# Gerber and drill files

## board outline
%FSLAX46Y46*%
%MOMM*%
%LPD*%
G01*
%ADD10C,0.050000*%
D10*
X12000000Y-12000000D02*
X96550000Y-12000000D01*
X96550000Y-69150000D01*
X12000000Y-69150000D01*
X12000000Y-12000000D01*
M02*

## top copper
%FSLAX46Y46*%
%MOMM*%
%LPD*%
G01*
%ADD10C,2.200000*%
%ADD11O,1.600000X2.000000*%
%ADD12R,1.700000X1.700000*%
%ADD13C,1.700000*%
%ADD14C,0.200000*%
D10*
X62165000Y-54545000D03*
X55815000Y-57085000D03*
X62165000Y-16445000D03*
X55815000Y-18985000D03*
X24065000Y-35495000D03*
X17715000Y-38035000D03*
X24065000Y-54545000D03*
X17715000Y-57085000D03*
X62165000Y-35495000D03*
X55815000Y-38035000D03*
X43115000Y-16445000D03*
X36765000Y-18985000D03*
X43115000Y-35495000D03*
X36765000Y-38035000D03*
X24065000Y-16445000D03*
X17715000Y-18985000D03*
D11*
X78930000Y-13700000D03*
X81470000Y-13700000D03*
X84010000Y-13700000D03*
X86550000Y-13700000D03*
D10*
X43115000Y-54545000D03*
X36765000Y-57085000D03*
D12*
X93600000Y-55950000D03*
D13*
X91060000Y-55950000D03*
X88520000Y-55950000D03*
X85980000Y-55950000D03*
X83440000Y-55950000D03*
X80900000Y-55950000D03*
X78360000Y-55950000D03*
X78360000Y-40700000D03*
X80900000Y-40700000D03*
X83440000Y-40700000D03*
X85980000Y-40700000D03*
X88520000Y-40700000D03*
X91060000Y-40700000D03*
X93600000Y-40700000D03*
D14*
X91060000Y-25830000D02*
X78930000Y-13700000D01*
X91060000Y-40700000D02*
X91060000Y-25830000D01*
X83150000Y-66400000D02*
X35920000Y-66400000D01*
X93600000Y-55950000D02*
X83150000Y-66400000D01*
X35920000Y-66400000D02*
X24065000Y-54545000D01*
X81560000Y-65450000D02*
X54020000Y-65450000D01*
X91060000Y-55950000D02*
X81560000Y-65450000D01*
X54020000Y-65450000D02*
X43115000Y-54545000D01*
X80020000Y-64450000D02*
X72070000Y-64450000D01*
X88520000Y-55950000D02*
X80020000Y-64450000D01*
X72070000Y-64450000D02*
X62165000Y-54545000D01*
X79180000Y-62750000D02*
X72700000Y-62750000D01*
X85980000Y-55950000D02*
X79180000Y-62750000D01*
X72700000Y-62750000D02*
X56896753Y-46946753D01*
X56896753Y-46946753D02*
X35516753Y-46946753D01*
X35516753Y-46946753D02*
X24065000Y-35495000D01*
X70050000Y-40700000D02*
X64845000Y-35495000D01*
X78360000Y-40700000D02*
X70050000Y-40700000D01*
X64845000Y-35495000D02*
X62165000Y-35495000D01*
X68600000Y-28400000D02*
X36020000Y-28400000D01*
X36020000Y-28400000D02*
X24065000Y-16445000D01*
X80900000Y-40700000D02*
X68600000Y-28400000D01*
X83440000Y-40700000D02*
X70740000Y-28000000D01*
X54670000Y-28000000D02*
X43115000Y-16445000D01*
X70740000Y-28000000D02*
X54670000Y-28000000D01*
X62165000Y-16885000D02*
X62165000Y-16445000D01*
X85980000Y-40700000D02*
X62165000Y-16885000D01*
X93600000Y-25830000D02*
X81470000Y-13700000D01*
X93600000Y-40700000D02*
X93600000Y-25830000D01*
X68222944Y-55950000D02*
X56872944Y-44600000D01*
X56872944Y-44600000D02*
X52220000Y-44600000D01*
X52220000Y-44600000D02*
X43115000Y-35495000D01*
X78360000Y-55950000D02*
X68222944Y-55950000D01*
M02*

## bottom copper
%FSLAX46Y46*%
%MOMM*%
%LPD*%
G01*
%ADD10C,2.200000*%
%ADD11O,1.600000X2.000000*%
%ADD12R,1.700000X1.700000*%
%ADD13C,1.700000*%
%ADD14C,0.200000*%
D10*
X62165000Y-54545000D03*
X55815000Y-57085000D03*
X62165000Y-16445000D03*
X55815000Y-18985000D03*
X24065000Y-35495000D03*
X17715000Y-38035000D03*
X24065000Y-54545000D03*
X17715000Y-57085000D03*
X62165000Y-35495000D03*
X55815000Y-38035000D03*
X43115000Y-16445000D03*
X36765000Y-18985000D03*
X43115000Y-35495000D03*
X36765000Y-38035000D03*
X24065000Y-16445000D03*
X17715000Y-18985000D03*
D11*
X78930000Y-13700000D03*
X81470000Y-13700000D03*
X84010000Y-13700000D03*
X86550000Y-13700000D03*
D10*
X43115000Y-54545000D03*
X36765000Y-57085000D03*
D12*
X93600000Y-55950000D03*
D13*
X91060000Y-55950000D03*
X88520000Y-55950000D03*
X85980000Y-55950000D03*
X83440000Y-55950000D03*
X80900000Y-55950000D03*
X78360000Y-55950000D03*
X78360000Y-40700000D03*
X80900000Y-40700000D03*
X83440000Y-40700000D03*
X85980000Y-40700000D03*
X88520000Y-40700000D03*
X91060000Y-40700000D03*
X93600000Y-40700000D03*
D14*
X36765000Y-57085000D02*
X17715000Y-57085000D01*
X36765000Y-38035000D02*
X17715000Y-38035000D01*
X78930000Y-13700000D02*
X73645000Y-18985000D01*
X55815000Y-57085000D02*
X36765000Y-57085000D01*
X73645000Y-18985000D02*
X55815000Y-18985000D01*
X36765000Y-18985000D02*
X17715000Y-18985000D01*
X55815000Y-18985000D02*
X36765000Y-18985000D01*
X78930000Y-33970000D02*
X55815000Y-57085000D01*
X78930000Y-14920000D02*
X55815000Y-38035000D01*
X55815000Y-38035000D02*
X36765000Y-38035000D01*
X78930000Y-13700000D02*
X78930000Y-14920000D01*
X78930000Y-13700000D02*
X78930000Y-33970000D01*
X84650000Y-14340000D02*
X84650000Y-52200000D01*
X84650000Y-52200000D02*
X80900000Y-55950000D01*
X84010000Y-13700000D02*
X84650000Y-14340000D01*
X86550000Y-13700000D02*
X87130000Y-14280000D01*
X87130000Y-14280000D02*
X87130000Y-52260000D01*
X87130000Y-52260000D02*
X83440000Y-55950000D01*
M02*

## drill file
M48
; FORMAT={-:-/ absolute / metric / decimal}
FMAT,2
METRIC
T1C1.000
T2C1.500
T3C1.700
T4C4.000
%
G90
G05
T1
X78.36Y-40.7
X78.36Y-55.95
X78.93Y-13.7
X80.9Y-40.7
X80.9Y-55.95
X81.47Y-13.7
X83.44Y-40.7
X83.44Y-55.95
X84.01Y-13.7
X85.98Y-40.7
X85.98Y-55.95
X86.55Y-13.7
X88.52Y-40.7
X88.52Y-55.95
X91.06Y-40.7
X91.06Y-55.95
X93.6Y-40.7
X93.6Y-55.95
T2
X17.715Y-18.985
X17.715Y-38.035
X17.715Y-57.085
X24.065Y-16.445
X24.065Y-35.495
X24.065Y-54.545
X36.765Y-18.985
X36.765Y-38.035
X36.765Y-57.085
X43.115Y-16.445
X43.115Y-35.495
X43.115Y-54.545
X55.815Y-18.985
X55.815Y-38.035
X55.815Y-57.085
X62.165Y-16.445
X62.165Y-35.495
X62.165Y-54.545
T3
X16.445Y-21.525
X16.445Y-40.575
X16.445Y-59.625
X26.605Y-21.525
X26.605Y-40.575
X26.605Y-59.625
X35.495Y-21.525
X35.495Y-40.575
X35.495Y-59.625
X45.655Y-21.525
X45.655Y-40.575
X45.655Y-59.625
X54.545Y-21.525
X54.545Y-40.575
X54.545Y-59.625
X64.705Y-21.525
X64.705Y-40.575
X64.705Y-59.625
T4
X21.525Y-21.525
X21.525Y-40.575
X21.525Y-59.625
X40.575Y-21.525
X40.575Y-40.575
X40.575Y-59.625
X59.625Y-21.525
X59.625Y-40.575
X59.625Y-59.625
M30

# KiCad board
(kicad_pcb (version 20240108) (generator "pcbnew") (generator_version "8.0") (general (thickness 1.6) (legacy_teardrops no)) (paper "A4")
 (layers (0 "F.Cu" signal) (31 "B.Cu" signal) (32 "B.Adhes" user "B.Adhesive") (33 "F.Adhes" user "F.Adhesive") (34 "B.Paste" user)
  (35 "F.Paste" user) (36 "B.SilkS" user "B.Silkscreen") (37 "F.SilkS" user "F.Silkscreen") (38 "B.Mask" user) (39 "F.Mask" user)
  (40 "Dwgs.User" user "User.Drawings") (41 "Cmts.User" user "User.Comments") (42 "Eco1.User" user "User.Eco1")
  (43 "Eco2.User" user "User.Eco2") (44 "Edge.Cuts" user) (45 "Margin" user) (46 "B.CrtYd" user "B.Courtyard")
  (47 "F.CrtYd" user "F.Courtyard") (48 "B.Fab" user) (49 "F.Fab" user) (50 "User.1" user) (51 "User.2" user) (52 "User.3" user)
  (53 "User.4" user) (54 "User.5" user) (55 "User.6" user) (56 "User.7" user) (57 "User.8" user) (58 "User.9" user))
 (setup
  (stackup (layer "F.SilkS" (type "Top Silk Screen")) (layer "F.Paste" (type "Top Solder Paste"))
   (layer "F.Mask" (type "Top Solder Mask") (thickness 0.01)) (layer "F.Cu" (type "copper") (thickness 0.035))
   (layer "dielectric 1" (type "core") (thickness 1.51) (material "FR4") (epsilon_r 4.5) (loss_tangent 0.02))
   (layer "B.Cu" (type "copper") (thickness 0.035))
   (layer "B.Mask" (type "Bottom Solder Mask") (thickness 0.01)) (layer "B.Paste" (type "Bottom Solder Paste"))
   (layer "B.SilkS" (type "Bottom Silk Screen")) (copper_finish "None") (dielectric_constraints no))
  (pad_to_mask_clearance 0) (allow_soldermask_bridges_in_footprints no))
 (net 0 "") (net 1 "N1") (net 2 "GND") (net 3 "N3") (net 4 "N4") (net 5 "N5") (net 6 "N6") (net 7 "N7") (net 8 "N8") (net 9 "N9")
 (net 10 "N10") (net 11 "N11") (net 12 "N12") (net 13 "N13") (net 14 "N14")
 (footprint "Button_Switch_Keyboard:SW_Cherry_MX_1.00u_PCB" (layer "F.Cu") (at 62.165 54.545)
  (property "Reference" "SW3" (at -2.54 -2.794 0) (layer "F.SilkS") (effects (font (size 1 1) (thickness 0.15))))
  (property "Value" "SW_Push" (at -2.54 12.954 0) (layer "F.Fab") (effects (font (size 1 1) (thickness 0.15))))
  (pad "" np_thru_hole circle (at -7.62 5.08) (size 1.7 1.7) (drill 1.7) (layers "*.Cu" "*.Mask"))
  (pad "" np_thru_hole circle (at -2.54 5.08) (size 4 4) (drill 4) (layers "*.Cu" "*.Mask"))
  (pad "" np_thru_hole circle (at 2.54 5.08) (size 1.7 1.7) (drill 1.7) (layers "*.Cu" "*.Mask"))
  (pad "1" thru_hole circle (at 0 0) (size 2.2 2.2) (drill 1.5) (layers "*.Cu" "*.Mask") (remove_unused_layers no) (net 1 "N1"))
  (pad "2" thru_hole circle (at -6.35 2.54) (size 2.2 2.2) (drill 1.5) (layers "*.Cu" "*.Mask") (remove_unused_layers no) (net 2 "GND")))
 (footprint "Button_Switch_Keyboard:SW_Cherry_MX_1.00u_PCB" (layer "F.Cu") (at 62.165 16.445)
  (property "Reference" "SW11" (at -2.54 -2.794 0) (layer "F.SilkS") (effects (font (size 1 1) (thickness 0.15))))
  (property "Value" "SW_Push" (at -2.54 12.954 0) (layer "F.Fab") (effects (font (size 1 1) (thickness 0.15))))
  (pad "" np_thru_hole circle (at -7.62 5.08) (size 1.7 1.7) (drill 1.7) (layers "*.Cu" "*.Mask"))
  (pad "" np_thru_hole circle (at -2.54 5.08) (size 4 4) (drill 4) (layers "*.Cu" "*.Mask"))
  (pad "" np_thru_hole circle (at 2.54 5.08) (size 1.7 1.7) (drill 1.7) (layers "*.Cu" "*.Mask"))
  (pad "1" thru_hole circle (at 0 0) (size 2.2 2.2) (drill 1.5) (layers "*.Cu" "*.Mask") (remove_unused_layers no) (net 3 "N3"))
  (pad "2" thru_hole circle (at -6.35 2.54) (size 2.2 2.2) (drill 1.5) (layers "*.Cu" "*.Mask") (remove_unused_layers no) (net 2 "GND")))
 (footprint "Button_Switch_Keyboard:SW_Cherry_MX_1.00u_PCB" (layer "F.Cu") (at 24.065 35.495)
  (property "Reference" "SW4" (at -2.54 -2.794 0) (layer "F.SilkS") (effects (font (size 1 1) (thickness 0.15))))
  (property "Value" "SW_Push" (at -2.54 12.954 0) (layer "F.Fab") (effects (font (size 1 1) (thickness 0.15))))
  (pad "" np_thru_hole circle (at -7.62 5.08) (size 1.7 1.7) (drill 1.7) (layers "*.Cu" "*.Mask"))
  (pad "" np_thru_hole circle (at -2.54 5.08) (size 4 4) (drill 4) (layers "*.Cu" "*.Mask"))
  (pad "" np_thru_hole circle (at 2.54 5.08) (size 1.7 1.7) (drill 1.7) (layers "*.Cu" "*.Mask"))
  (pad "1" thru_hole circle (at 0 0) (size 2.2 2.2) (drill 1.5) (layers "*.Cu" "*.Mask") (remove_unused_layers no) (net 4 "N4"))
  (pad "2" thru_hole circle (at -6.35 2.54) (size 2.2 2.2) (drill 1.5) (layers "*.Cu" "*.Mask") (remove_unused_layers no) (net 2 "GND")))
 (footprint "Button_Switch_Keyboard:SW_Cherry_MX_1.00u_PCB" (layer "F.Cu") (at 24.065 54.545)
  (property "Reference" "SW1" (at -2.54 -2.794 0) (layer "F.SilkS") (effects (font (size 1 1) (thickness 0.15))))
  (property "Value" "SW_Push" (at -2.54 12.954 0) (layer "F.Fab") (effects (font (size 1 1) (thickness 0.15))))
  (pad "" np_thru_hole circle (at -7.62 5.08) (size 1.7 1.7) (drill 1.7) (layers "*.Cu" "*.Mask"))
  (pad "" np_thru_hole circle (at -2.54 5.08) (size 4 4) (drill 4) (layers "*.Cu" "*.Mask"))
  (pad "" np_thru_hole circle (at 2.54 5.08) (size 1.7 1.7) (drill 1.7) (layers "*.Cu" "*.Mask"))
  (pad "1" thru_hole circle (at 0 0) (size 2.2 2.2) (drill 1.5) (layers "*.Cu" "*.Mask") (remove_unused_layers no) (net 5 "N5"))
  (pad "2" thru_hole circle (at -6.35 2.54) (size 2.2 2.2) (drill 1.5) (layers "*.Cu" "*.Mask") (remove_unused_layers no) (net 2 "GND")))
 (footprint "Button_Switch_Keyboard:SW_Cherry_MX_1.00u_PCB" (layer "F.Cu") (at 62.165 35.495)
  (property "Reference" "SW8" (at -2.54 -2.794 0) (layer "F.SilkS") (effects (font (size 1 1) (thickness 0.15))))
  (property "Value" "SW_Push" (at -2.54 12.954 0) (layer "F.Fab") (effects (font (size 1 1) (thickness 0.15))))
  (pad "" np_thru_hole circle (at -7.62 5.08) (size 1.7 1.7) (drill 1.7) (layers "*.Cu" "*.Mask"))
  (pad "" np_thru_hole circle (at -2.54 5.08) (size 4 4) (drill 4) (layers "*.Cu" "*.Mask"))
  (pad "" np_thru_hole circle (at 2.54 5.08) (size 1.7 1.7) (drill 1.7) (layers "*.Cu" "*.Mask"))
  (pad "1" thru_hole circle (at 0 0) (size 2.2 2.2) (drill 1.5) (layers "*.Cu" "*.Mask") (remove_unused_layers no) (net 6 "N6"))
  (pad "2" thru_hole circle (at -6.35 2.54) (size 2.2 2.2) (drill 1.5) (layers "*.Cu" "*.Mask") (remove_unused_layers no) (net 2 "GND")))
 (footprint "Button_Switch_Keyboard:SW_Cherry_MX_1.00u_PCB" (layer "F.Cu") (at 43.115 16.445)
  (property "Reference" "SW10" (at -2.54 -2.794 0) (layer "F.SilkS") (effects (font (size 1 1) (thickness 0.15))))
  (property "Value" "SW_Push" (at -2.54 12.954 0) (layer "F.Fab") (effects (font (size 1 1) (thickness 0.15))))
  (pad "" np_thru_hole circle (at -7.62 5.08) (size 1.7 1.7) (drill 1.7) (layers "*.Cu" "*.Mask"))
  (pad "" np_thru_hole circle (at -2.54 5.08) (size 4 4) (drill 4) (layers "*.Cu" "*.Mask"))
  (pad "" np_thru_hole circle (at 2.54 5.08) (size 1.7 1.7) (drill 1.7) (layers "*.Cu" "*.Mask"))
  (pad "1" thru_hole circle (at 0 0) (size 2.2 2.2) (drill 1.5) (layers "*.Cu" "*.Mask") (remove_unused_layers no) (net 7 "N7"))
  (pad "2" thru_hole circle (at -6.35 2.54) (size 2.2 2.2) (drill 1.5) (layers "*.Cu" "*.Mask") (remove_unused_layers no) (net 2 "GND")))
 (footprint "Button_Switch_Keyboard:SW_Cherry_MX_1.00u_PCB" (layer "F.Cu") (at 43.115 35.495)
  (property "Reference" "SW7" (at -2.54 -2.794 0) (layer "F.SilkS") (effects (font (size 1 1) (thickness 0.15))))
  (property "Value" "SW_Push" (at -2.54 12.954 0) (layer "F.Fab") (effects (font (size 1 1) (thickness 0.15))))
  (pad "" np_thru_hole circle (at -7.62 5.08) (size 1.7 1.7) (drill 1.7) (layers "*.Cu" "*.Mask"))
  (pad "" np_thru_hole circle (at -2.54 5.08) (size 4 4) (drill 4) (layers "*.Cu" "*.Mask"))
  (pad "" np_thru_hole circle (at 2.54 5.08) (size 1.7 1.7) (drill 1.7) (layers "*.Cu" "*.Mask"))
  (pad "1" thru_hole circle (at 0 0) (size 2.2 2.2) (drill 1.5) (layers "*.Cu" "*.Mask") (remove_unused_layers no) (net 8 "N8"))
  (pad "2" thru_hole circle (at -6.35 2.54) (size 2.2 2.2) (drill 1.5) (layers "*.Cu" "*.Mask") (remove_unused_layers no) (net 2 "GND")))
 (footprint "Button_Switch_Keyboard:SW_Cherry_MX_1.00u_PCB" (layer "F.Cu") (at 24.065 16.445)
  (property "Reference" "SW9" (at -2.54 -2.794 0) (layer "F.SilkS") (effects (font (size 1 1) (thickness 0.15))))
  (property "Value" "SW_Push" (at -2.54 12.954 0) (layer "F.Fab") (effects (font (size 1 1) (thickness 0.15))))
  (pad "" np_thru_hole circle (at -7.62 5.08) (size 1.7 1.7) (drill 1.7) (layers "*.Cu" "*.Mask"))
  (pad "" np_thru_hole circle (at -2.54 5.08) (size 4 4) (drill 4) (layers "*.Cu" "*.Mask"))
  (pad "" np_thru_hole circle (at 2.54 5.08) (size 1.7 1.7) (drill 1.7) (layers "*.Cu" "*.Mask"))
  (pad "1" thru_hole circle (at 0 0) (size 2.2 2.2) (drill 1.5) (layers "*.Cu" "*.Mask") (remove_unused_layers no) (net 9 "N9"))
  (pad "2" thru_hole circle (at -6.35 2.54) (size 2.2 2.2) (drill 1.5) (layers "*.Cu" "*.Mask") (remove_unused_layers no) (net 2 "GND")))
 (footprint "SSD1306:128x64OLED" (layer "F.Cu") (at 82.55 24.3)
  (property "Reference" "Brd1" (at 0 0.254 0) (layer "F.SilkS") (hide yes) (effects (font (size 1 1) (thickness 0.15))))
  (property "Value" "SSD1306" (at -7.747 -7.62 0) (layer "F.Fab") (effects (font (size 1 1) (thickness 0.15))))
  (pad "1" thru_hole oval (at -3.62 -10.6 90) (size 2 1.6) (drill 1) (layers "*.Cu" "*.Mask") (remove_unused_layers no) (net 2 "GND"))
  (pad "2" thru_hole oval (at -1.08 -10.6 90) (size 2 1.6) (drill 1) (layers "*.Cu" "*.Mask") (remove_unused_layers no) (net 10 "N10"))
  (pad "3" thru_hole oval (at 1.46 -10.6 90) (size 2 1.6) (drill 1) (layers "*.Cu" "*.Mask") (remove_unused_layers no) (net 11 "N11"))
  (pad "4" thru_hole oval (at 4 -10.6 90) (size 2 1.6) (drill 1) (layers "*.Cu" "*.Mask") (remove_unused_layers no) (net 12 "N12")))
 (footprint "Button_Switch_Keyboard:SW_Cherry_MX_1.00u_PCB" (layer "F.Cu") (at 43.115 54.545)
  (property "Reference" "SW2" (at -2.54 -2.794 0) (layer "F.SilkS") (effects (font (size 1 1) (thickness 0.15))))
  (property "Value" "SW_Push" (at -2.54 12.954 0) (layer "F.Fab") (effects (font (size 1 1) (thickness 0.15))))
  (pad "" np_thru_hole circle (at -7.62 5.08) (size 1.7 1.7) (drill 1.7) (layers "*.Cu" "*.Mask"))
  (pad "" np_thru_hole circle (at -2.54 5.08) (size 4 4) (drill 4) (layers "*.Cu" "*.Mask"))
  (pad "" np_thru_hole circle (at 2.54 5.08) (size 1.7 1.7) (drill 1.7) (layers "*.Cu" "*.Mask"))
  (pad "1" thru_hole circle (at 0 0) (size 2.2 2.2) (drill 1.5) (layers "*.Cu" "*.Mask") (remove_unused_layers no) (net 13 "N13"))
  (pad "2" thru_hole circle (at -6.35 2.54) (size 2.2 2.2) (drill 1.5) (layers "*.Cu" "*.Mask") (remove_unused_layers no) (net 2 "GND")))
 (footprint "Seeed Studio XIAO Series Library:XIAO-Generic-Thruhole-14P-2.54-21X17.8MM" (layer "B.Cu") (at 85.98 48.325 90)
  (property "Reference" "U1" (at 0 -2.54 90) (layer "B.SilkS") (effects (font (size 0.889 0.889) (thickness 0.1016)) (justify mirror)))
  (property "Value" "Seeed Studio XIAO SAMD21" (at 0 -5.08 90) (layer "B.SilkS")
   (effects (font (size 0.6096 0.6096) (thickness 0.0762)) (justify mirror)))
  (pad "1" thru_hole rect (at -7.625 7.62 90) (size 1.7 1.7) (drill 1) (layers "*.Cu" "*.Mask") (remove_unused_layers no) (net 5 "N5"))
  (pad "2" thru_hole circle (at -7.625 5.08 90) (size 1.7 1.7) (drill 1) (layers "*.Cu" "*.Mask") (remove_unused_layers no) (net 13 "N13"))
  (pad "3" thru_hole circle (at -7.625 2.54 90) (size 1.7 1.7) (drill 1) (layers "*.Cu" "*.Mask") (remove_unused_layers no) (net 1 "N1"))
  (pad "4" thru_hole circle (at -7.625 0 90) (size 1.7 1.7) (drill 1) (layers "*.Cu" "*.Mask") (remove_unused_layers no) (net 4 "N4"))
  (pad "5" thru_hole circle (at -7.625 -2.54 90) (size 1.7 1.7) (drill 1) (layers "*.Cu" "*.Mask") (remove_unused_layers no) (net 12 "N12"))
  (pad "6" thru_hole circle (at -7.625 -5.08 270) (size 1.7 1.7) (drill 1) (layers "*.Cu" "*.Mask") (remove_unused_layers no) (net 11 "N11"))
  (pad "7" thru_hole circle (at -7.625 -7.62 90) (size 1.7 1.7) (drill 1) (layers "*.Cu" "*.Mask") (remove_unused_layers no) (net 8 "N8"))
  (pad "8" thru_hole circle (at 7.625 -7.62 90) (size 1.7 1.7) (drill 1) (layers "*.Cu" "*.Mask") (remove_unused_layers no) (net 6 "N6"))
  (pad "9" thru_hole circle (at 7.625 -5.08 90) (size 1.7 1.7) (drill 1) (layers "*.Cu" "*.Mask") (remove_unused_layers no) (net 9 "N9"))
  (pad "10" thru_hole circle (at 7.625 -2.54 90) (size 1.7 1.7) (drill 1) (layers "*.Cu" "*.Mask") (remove_unused_layers no) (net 7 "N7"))
  (pad "11" thru_hole circle (at 7.625 0 90) (size 1.7 1.7) (drill 1) (layers "*.Cu" "*.Mask") (remove_unused_layers no) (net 3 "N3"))
  (pad "12" thru_hole circle (at 7.625 2.54 90) (size 1.7 1.7) (drill 1) (layers "*.Cu" "*.Mask") (remove_unused_layers no) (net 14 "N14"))
  (pad "13" thru_hole circle (at 7.625 5.08 90) (size 1.7 1.7) (drill 1) (layers "*.Cu" "*.Mask") (remove_unused_layers no) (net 2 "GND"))
  (pad "14" thru_hole circle (at 7.625 7.62 90) (size 1.7 1.7) (drill 1) (layers "*.Cu" "*.Mask") (remove_unused_layers no) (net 10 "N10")))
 (gr_rect (start 12 12) (end 96.55 69.15) (stroke (width 0.05) (type default)) (fill none) (layer "Edge.Cuts"))
 (segment (start 91.06 25.83) (end 78.93 13.7) (width 0.2) (layer "F.Cu") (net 2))
 (segment (start 91.06 40.7) (end 91.06 25.83) (width 0.2) (layer "F.Cu") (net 2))
 (segment (start 36.765 57.085) (end 17.715 57.085) (width 0.2) (layer "B.Cu") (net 2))
 (segment (start 36.765 38.035) (end 17.715 38.035) (width 0.2) (layer "B.Cu") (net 2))
 (segment (start 78.93 13.7) (end 73.645 18.985) (width 0.2) (layer "B.Cu") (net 2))
 (segment (start 55.815 57.085) (end 36.765 57.085) (width 0.2) (layer "B.Cu") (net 2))
 (segment (start 73.645 18.985) (end 55.815 18.985) (width 0.2) (layer "B.Cu") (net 2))
 (segment (start 36.765 18.985) (end 17.715 18.985) (width 0.2) (layer "B.Cu") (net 2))
 (segment (start 55.815 18.985) (end 36.765 18.985) (width 0.2) (layer "B.Cu") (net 2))
 (segment (start 78.93 33.97) (end 55.815 57.085) (width 0.2) (layer "B.Cu") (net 2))
 (segment (start 78.93 14.92) (end 55.815 38.035) (width 0.2) (layer "B.Cu") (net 2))
 (segment (start 55.815 38.035) (end 36.765 38.035) (width 0.2) (layer "B.Cu") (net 2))
 (segment (start 78.93 13.7) (end 78.93 14.92) (width 0.2) (layer "B.Cu") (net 2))
 (segment (start 78.93 13.7) (end 78.93 33.97) (width 0.2) (layer "B.Cu") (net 2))
 (segment (start 84.65 14.34) (end 84.65 52.2) (width 0.2) (layer "B.Cu") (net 11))
 (segment (start 84.65 52.2) (end 80.9 55.95) (width 0.2) (layer "B.Cu") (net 11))
 (segment (start 84.01 13.7) (end 84.65 14.34) (width 0.2) (layer "B.Cu") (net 11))
 (segment (start 83.15 66.4) (end 35.92 66.4) (width 0.2) (layer "F.Cu") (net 5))
 (segment (start 93.6 55.95) (end 83.15 66.4) (width 0.2) (layer "F.Cu") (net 5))
 (segment (start 35.92 66.4) (end 24.065 54.545) (width 0.2) (layer "F.Cu") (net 5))
 (segment (start 81.56 65.45) (end 54.02 65.45) (width 0.2) (layer "F.Cu") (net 13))
 (segment (start 91.06 55.95) (end 81.56 65.45) (width 0.2) (layer "F.Cu") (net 13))
 (segment (start 54.02 65.45) (end 43.115 54.545) (width 0.2) (layer "F.Cu") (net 13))
 (segment (start 80.02 64.45) (end 72.07 64.45) (width 0.2) (layer "F.Cu") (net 1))
 (segment (start 88.52 55.95) (end 80.02 64.45) (width 0.2) (layer "F.Cu") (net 1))
 (segment (start 72.07 64.45) (end 62.165 54.545) (width 0.2) (layer "F.Cu") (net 1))
 (segment (start 79.18 62.75) (end 72.7 62.75) (width 0.2) (layer "F.Cu") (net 4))
 (segment (start 85.98 55.95) (end 79.18 62.75) (width 0.2) (layer "F.Cu") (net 4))
 (segment (start 72.7 62.75) (end 56.896753 46.946753) (width 0.2) (layer "F.Cu") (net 4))
 (segment (start 56.896753 46.946753) (end 35.516753 46.946753) (width 0.2) (layer "F.Cu") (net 4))
 (segment (start 35.516753 46.946753) (end 24.065 35.495) (width 0.2) (layer "F.Cu") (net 4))
 (segment (start 70.05 40.7) (end 64.845 35.495) (width 0.2) (layer "F.Cu") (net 6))
 (segment (start 78.36 40.7) (end 70.05 40.7) (width 0.2) (layer "F.Cu") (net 6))
 (segment (start 64.845 35.495) (end 62.165 35.495) (width 0.2) (layer "F.Cu") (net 6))
 (segment (start 68.6 28.4) (end 36.02 28.4) (width 0.2) (layer "F.Cu") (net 9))
 (segment (start 36.02 28.4) (end 24.065 16.445) (width 0.2) (layer "F.Cu") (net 9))
 (segment (start 80.9 40.7) (end 68.6 28.4) (width 0.2) (layer "F.Cu") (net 9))
 (segment (start 83.44 40.7) (end 70.74 28) (width 0.2) (layer "F.Cu") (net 7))
 (segment (start 54.67 28) (end 43.115 16.445) (width 0.2) (layer "F.Cu") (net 7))
 (segment (start 70.74 28) (end 54.67 28) (width 0.2) (layer "F.Cu") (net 7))
 (segment (start 62.165 16.885) (end 62.165 16.445) (width 0.2) (layer "F.Cu") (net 3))
 (segment (start 85.98 40.7) (end 62.165 16.885) (width 0.2) (layer "F.Cu") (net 3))
 (segment (start 86.55 13.7) (end 87.13 14.28) (width 0.2) (layer "B.Cu") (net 12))
 (segment (start 87.13 14.28) (end 87.13 52.26) (width 0.2) (layer "B.Cu") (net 12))
 (segment (start 87.13 52.26) (end 83.44 55.95) (width 0.2) (layer "B.Cu") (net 12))
 (segment (start 93.6 25.83) (end 81.47 13.7) (width 0.2) (layer "F.Cu") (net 10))
 (segment (start 93.6 40.7) (end 93.6 25.83) (width 0.2) (layer "F.Cu") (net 10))
 (segment (start 68.222944 55.95) (end 56.872944 44.6) (width 0.2) (layer "F.Cu") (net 8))
 (segment (start 56.872944 44.6) (end 52.22 44.6) (width 0.2) (layer "F.Cu") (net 8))
 (segment (start 52.22 44.6) (end 43.115 35.495) (width 0.2) (layer "F.Cu") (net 8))
 (segment (start 78.36 55.95) (end 68.222944 55.95) (width 0.2) (layer "F.Cu") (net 8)))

